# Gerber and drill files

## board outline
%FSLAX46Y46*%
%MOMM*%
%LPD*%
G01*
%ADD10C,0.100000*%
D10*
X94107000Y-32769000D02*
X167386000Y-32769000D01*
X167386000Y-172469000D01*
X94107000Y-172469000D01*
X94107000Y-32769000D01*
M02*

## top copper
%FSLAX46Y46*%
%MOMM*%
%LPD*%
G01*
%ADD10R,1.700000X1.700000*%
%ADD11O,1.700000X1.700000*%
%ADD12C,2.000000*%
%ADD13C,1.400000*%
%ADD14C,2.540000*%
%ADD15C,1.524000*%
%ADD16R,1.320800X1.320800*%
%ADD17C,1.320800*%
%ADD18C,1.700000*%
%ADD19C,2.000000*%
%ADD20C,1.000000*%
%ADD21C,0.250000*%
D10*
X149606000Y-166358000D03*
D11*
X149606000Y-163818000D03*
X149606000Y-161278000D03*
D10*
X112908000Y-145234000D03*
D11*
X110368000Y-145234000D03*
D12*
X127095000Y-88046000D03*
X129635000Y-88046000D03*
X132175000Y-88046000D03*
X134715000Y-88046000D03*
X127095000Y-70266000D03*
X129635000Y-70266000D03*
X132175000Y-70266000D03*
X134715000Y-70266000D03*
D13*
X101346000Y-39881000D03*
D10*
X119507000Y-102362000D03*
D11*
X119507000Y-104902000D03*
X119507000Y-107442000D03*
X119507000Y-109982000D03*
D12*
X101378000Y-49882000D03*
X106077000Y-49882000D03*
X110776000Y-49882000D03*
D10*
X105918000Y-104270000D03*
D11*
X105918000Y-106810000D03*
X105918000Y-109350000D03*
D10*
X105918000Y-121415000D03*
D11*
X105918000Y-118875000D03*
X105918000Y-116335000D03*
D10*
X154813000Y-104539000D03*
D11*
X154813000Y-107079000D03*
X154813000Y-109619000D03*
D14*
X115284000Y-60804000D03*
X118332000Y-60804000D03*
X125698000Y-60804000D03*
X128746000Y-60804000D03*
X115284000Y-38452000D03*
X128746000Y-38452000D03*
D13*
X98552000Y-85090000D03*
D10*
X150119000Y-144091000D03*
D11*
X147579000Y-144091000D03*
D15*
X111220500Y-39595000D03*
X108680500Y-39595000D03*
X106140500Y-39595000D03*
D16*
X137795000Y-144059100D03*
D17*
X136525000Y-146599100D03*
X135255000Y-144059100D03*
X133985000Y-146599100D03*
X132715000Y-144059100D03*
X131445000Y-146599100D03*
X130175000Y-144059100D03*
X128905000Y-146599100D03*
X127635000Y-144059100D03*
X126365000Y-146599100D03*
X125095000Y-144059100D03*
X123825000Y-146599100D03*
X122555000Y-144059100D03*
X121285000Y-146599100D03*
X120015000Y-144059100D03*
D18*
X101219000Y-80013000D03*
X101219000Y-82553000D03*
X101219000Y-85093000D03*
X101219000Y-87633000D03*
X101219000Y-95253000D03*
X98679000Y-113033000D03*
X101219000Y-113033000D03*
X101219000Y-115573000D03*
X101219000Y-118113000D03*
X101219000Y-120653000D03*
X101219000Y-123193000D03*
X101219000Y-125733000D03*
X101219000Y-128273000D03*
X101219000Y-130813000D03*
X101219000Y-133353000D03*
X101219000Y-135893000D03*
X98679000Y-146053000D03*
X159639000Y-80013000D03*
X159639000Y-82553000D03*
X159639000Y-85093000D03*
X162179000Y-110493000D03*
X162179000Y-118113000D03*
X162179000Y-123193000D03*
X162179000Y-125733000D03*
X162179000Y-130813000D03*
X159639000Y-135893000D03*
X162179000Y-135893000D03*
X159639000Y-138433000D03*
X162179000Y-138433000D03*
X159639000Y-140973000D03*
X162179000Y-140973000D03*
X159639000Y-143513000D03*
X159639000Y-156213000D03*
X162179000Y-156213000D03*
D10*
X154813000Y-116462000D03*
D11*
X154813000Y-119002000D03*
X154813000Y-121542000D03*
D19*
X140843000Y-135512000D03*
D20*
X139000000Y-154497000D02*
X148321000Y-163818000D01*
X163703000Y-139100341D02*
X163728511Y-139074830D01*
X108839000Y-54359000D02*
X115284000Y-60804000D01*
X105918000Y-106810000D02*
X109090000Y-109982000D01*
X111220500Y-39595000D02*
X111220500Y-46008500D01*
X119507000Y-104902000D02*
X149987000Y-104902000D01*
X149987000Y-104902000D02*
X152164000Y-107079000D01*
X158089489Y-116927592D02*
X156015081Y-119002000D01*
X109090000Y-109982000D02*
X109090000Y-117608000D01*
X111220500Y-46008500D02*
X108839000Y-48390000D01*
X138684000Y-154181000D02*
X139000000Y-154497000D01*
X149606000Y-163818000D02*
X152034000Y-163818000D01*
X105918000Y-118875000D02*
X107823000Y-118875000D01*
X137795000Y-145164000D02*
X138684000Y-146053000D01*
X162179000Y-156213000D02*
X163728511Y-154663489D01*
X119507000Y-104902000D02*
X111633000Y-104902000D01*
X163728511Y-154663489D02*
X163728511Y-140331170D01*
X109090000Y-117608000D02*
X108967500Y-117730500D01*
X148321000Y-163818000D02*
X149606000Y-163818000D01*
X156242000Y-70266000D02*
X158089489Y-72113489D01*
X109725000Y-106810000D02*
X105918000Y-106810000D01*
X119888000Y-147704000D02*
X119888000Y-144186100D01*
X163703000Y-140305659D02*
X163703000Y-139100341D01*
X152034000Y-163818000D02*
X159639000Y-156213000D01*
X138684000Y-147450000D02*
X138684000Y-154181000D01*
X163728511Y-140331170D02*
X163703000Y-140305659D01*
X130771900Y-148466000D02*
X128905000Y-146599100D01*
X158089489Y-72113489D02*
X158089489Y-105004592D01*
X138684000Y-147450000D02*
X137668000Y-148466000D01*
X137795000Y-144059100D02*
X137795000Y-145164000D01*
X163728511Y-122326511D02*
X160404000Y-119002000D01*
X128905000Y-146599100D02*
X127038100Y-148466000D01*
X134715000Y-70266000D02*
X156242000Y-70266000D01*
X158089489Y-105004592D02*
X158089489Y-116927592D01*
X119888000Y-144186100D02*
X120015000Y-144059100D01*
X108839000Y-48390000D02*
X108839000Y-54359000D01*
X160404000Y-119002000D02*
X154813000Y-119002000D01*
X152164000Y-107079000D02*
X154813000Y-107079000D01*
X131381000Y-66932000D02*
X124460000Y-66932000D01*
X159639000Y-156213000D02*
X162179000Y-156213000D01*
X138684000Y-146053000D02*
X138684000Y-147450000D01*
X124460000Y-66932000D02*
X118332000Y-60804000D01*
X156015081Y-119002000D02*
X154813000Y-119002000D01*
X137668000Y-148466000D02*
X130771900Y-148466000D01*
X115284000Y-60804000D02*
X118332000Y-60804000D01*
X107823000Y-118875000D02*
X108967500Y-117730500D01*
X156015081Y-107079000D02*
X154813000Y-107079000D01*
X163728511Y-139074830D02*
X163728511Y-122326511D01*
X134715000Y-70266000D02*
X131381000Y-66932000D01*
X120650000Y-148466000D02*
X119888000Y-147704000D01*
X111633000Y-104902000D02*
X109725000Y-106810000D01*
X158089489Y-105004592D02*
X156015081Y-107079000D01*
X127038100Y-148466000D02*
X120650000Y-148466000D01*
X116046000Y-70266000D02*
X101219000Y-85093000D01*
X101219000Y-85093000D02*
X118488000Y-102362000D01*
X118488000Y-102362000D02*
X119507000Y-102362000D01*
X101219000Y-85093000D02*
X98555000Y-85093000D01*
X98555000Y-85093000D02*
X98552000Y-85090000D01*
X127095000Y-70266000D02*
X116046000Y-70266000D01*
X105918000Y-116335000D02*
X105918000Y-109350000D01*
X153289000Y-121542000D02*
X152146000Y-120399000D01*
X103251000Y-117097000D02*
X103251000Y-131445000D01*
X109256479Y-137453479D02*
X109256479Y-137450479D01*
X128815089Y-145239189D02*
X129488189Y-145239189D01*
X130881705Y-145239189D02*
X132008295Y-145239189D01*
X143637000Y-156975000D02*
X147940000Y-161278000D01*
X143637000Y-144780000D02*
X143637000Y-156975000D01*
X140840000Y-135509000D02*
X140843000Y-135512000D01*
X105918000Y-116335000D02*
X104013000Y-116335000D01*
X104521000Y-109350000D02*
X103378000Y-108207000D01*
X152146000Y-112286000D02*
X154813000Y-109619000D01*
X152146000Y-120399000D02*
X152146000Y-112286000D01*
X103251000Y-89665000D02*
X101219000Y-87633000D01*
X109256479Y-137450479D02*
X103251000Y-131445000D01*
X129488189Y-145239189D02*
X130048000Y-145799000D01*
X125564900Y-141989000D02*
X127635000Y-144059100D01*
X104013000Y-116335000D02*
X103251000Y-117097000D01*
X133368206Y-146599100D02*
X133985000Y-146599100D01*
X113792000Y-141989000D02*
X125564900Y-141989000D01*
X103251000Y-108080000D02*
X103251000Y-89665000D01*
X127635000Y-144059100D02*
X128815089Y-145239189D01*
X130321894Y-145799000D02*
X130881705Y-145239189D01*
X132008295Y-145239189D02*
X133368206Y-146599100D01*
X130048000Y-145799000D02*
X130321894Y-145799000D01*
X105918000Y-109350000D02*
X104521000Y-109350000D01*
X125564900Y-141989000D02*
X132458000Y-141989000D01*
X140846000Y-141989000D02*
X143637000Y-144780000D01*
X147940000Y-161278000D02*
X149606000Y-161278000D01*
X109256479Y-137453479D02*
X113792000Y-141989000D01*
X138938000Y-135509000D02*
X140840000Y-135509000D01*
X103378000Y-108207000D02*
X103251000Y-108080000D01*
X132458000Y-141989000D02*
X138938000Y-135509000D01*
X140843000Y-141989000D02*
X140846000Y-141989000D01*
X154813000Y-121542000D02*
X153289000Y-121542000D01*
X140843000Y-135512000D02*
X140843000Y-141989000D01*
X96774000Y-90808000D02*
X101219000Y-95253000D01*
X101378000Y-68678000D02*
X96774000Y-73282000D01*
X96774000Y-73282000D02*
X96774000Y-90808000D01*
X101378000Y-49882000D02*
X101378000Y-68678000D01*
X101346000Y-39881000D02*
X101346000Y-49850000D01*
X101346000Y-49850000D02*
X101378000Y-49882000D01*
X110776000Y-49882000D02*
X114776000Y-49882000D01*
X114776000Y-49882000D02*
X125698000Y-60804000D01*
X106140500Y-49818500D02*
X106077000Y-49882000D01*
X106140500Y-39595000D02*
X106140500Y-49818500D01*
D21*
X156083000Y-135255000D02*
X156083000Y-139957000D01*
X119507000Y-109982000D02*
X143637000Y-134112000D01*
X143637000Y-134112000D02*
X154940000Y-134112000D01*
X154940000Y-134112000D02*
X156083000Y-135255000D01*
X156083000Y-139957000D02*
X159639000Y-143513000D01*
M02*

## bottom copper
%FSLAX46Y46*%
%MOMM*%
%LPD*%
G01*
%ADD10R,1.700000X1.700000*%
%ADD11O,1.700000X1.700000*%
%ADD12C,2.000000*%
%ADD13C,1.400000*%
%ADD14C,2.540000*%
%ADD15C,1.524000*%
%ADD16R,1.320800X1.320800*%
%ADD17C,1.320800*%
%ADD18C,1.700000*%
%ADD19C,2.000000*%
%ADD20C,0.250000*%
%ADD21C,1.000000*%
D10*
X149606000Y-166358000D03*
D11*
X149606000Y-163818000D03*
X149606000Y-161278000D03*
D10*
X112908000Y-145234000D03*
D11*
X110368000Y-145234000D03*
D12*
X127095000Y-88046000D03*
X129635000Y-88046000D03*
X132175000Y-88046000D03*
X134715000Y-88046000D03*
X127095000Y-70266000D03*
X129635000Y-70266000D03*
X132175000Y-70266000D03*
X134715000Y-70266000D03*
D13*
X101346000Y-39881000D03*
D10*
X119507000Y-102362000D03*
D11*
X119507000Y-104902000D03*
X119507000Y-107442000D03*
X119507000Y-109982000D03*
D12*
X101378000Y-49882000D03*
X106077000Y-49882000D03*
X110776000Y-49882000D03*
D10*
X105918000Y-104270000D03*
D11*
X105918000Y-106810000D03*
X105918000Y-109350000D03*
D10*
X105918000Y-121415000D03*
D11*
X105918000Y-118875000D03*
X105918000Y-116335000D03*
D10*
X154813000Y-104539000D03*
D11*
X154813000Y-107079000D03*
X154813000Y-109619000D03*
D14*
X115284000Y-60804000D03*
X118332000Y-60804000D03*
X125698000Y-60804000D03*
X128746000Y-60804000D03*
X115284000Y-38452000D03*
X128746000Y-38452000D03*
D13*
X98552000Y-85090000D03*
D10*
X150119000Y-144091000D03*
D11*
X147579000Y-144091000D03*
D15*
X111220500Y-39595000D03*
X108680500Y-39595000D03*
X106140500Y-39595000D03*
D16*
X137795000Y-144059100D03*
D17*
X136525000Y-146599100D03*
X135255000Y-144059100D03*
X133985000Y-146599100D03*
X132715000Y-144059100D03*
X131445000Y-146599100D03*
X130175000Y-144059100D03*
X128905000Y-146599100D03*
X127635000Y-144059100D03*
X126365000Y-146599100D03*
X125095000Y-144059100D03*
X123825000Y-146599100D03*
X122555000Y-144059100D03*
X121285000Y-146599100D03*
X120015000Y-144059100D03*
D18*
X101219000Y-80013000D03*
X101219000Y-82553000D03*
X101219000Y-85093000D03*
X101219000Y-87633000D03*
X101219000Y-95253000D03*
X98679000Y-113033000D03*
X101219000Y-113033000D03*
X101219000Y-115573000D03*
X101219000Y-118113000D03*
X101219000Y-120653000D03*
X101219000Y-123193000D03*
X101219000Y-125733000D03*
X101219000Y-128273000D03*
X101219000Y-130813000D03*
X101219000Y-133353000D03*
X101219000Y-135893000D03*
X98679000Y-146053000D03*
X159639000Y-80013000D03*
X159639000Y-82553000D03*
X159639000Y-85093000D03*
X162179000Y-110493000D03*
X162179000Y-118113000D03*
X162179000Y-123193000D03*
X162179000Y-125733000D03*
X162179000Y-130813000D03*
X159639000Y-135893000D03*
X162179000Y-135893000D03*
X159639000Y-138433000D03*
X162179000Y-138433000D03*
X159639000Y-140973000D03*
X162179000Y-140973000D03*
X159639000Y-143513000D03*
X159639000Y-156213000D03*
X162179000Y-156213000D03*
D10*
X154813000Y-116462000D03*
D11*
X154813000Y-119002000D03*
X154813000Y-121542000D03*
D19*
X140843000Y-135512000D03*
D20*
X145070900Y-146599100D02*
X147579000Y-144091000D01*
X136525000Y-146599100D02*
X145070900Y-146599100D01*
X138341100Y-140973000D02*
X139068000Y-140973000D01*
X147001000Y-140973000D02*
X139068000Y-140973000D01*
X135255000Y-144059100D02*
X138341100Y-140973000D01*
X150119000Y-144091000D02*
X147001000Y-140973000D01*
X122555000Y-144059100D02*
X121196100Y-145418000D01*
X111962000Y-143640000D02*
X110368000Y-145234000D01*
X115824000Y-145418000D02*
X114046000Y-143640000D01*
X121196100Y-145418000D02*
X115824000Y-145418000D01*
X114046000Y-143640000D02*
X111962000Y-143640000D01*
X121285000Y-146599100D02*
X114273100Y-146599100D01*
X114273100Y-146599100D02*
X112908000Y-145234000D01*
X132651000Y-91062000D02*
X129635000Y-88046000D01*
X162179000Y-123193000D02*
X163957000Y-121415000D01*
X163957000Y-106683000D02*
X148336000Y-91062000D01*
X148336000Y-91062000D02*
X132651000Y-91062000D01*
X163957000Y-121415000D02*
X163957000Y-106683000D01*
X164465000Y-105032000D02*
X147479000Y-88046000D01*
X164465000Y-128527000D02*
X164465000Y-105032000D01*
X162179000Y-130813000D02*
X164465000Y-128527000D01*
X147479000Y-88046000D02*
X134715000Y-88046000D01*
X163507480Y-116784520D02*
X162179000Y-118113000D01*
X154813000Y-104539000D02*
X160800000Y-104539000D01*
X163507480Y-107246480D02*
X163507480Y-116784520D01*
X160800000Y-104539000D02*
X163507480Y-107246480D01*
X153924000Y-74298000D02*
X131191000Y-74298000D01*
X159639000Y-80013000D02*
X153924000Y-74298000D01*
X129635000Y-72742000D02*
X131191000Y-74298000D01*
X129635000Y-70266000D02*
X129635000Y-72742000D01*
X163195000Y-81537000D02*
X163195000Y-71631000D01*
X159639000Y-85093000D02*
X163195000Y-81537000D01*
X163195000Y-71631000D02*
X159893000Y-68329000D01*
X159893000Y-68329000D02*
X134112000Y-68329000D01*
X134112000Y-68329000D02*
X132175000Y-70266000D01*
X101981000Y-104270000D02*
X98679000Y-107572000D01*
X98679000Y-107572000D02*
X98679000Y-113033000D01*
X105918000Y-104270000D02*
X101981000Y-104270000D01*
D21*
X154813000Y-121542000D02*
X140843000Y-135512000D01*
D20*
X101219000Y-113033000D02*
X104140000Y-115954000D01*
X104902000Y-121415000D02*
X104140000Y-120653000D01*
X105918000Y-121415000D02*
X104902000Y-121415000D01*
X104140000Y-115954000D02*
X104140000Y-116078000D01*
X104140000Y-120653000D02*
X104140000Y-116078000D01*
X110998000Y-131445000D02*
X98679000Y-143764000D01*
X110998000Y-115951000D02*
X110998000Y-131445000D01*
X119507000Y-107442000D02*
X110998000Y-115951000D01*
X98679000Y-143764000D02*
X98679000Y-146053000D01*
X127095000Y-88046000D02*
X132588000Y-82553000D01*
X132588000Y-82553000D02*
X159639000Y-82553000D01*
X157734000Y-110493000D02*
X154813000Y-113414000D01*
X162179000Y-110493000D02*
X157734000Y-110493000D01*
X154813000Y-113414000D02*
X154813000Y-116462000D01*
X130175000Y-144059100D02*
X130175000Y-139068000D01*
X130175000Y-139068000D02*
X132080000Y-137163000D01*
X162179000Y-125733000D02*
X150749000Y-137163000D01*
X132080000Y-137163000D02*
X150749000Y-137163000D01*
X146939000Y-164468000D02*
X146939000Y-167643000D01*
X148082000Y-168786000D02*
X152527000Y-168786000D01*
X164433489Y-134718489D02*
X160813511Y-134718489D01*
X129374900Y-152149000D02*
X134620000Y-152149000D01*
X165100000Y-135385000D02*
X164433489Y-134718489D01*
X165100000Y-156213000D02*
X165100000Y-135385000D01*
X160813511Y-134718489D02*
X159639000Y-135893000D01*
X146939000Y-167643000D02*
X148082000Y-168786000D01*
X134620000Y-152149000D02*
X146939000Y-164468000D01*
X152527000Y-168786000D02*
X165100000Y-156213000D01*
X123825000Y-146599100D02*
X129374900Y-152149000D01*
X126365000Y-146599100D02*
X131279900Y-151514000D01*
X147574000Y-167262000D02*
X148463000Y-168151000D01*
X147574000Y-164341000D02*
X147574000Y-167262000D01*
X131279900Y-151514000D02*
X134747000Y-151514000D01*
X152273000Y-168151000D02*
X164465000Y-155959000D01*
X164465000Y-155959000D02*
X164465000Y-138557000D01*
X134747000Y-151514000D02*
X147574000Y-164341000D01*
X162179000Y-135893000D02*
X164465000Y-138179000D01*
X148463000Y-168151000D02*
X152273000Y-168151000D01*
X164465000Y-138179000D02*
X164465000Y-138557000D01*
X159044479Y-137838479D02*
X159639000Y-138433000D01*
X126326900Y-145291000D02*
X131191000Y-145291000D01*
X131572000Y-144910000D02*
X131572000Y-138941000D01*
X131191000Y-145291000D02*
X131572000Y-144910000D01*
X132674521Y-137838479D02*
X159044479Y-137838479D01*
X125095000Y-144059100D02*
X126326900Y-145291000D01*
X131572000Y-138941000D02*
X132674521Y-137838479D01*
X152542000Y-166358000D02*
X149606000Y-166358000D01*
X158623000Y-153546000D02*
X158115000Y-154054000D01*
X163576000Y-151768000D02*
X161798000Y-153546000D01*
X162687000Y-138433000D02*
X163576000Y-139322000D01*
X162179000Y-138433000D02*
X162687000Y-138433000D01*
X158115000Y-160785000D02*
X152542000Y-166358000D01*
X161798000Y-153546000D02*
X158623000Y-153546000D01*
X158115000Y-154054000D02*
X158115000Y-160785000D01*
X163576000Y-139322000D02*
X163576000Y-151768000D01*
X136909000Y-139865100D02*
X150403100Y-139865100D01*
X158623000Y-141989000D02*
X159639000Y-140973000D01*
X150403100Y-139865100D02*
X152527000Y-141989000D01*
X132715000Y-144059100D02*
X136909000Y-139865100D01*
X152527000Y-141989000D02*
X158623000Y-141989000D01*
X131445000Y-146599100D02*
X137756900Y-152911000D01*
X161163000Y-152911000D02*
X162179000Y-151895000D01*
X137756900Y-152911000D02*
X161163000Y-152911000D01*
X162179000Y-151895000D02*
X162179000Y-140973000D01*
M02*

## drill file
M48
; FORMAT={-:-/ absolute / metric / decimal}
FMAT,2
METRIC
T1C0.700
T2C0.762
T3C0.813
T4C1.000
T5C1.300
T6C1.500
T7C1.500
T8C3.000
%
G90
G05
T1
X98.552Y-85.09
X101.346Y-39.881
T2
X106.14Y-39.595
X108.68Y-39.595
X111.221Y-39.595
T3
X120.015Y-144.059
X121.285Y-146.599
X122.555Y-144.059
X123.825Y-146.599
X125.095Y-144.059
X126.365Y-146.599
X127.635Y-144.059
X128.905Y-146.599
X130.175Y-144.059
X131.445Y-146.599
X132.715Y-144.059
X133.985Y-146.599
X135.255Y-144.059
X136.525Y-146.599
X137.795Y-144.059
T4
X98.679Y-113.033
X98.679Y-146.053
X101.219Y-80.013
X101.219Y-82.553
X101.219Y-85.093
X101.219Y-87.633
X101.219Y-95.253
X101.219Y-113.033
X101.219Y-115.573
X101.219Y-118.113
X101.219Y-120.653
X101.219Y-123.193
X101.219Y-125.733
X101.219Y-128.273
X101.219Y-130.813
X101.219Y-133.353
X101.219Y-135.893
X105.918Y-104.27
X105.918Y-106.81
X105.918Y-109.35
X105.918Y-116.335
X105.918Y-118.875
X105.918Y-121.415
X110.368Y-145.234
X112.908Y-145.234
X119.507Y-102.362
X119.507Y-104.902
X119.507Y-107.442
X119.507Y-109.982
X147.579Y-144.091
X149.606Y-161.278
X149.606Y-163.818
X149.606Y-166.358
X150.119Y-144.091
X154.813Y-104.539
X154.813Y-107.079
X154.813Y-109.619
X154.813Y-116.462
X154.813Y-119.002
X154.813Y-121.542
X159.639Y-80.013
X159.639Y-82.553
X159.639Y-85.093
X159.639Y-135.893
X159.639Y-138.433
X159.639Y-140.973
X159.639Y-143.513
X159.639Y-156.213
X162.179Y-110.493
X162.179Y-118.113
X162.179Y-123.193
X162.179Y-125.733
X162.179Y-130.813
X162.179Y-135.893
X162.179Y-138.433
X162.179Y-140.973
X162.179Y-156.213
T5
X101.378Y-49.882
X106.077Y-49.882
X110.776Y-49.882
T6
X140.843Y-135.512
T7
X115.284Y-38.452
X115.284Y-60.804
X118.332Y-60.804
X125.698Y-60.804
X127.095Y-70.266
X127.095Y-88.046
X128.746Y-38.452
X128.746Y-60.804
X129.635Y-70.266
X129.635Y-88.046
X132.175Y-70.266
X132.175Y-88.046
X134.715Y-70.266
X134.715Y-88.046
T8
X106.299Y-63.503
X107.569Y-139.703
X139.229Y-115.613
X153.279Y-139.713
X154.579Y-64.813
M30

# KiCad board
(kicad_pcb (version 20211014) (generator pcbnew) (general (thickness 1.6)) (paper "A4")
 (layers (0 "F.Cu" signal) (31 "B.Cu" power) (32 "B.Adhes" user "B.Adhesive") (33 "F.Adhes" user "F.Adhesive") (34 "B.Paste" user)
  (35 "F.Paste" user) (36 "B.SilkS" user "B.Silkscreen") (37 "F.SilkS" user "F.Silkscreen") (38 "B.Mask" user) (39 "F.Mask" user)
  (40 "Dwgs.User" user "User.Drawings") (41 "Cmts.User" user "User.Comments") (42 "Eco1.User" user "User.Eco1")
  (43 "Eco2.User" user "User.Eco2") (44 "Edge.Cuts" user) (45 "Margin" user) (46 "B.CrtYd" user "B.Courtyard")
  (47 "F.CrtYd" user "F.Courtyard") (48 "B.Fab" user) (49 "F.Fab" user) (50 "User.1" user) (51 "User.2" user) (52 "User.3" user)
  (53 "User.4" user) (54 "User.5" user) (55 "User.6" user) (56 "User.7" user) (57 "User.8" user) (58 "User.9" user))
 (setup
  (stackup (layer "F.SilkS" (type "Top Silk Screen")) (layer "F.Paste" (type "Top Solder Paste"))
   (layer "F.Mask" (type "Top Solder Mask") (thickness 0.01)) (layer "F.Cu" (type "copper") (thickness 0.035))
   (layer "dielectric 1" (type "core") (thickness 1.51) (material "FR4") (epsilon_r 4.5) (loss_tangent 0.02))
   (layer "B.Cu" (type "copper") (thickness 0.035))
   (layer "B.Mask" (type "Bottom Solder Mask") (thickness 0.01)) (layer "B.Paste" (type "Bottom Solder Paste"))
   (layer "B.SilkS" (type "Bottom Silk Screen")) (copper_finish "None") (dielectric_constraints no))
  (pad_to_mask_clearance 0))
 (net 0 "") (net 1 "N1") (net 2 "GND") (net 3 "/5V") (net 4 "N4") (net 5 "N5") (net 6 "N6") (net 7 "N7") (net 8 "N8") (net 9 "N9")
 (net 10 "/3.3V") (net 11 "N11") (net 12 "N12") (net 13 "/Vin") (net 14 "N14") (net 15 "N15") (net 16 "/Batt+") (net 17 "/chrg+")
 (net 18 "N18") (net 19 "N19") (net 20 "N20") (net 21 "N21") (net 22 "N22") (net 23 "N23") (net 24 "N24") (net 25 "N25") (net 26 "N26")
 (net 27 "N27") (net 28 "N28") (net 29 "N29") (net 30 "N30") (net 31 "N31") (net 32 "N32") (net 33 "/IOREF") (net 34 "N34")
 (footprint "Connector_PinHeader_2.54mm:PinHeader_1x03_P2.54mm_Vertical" (layer "F.Cu") (at 149.606 166.358 180)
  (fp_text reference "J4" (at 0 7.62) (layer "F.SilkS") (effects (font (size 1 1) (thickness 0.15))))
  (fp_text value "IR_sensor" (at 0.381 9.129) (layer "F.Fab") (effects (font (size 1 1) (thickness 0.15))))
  (pad "1" thru_hole rect (at 0 0 180) (size 1.7 1.7) (drill 1) (layers *.Cu *.Mask) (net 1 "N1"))
  (pad "2" thru_hole oval (at 0 2.54 180) (size 1.7 1.7) (drill 1) (layers *.Cu *.Mask) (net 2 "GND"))
  (pad "3" thru_hole oval (at 0 5.08 180) (size 1.7 1.7) (drill 1) (layers *.Cu *.Mask) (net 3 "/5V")))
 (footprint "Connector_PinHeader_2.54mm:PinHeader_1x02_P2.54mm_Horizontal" (layer "F.Cu") (at 112.908 145.234 -90)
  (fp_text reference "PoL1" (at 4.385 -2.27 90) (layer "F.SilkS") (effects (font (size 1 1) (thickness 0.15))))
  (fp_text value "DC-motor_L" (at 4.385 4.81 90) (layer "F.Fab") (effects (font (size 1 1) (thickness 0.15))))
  (pad "1" thru_hole rect (at 0 0 270) (size 1.7 1.7) (drill 1) (layers *.Cu *.Mask) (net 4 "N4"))
  (pad "2" thru_hole oval (at 0 2.54 270) (size 1.7 1.7) (drill 1) (layers *.Cu *.Mask) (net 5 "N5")))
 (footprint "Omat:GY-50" (layer "F.Cu") (at 119.348 90.713)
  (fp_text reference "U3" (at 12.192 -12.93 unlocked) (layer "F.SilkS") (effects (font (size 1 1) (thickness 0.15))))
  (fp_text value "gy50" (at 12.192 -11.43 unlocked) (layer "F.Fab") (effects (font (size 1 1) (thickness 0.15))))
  (pad "1" thru_hole circle (at 7.747 -2.667) (size 2 2) (drill 1.5) (layers *.Cu *.Mask) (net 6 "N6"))
  (pad "2" thru_hole circle (at 10.287 -2.667) (size 2 2) (drill 1.5) (layers *.Cu *.Mask) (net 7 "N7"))
  (pad "3" thru_hole circle (at 12.827 -2.667) (size 2 2) (drill 1.5) (layers *.Cu *.Mask) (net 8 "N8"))
  (pad "4" thru_hole circle (at 15.367 -2.667) (size 2 2) (drill 1.5) (layers *.Cu *.Mask) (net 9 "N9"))
  (pad "5" thru_hole circle (at 7.747 -20.447) (size 2 2) (drill 1.5) (layers *.Cu *.Mask) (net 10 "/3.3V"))
  (pad "6" thru_hole circle (at 10.287 -20.447) (size 2 2) (drill 1.5) (layers *.Cu *.Mask) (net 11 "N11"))
  (pad "7" thru_hole circle (at 12.827 -20.447) (size 2 2) (drill 1.5) (layers *.Cu *.Mask) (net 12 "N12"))
  (pad "8" thru_hole circle (at 15.367 -20.447) (size 2 2) (drill 1.5) (layers *.Cu *.Mask) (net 2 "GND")))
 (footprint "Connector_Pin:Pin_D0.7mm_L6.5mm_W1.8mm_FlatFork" (layer "F.Cu") (at 101.346 39.881)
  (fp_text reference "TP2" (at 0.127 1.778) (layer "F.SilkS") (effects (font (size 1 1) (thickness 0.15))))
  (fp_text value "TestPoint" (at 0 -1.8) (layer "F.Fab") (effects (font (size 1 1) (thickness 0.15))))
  (pad "1" thru_hole circle (at 0 0) (size 1.4 1.4) (drill 0.7) (layers *.Cu *.Mask) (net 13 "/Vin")))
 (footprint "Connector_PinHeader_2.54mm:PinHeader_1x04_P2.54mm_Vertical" (layer "F.Cu") (at 119.507 102.362)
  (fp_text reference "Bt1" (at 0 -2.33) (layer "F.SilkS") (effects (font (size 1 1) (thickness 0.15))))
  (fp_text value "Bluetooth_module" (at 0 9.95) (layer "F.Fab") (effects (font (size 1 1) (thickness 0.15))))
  (pad "1" thru_hole rect (at 0 0) (size 1.7 1.7) (drill 1) (layers *.Cu *.Mask) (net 10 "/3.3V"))
  (pad "2" thru_hole oval (at 0 2.54) (size 1.7 1.7) (drill 1) (layers *.Cu *.Mask) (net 2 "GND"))
  (pad "3" thru_hole oval (at 0 5.08) (size 1.7 1.7) (drill 1) (layers *.Cu *.Mask) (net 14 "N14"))
  (pad "4" thru_hole oval (at 0 7.62) (size 1.7 1.7) (drill 1) (layers *.Cu *.Mask) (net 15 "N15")))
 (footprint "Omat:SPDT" (layer "F.Cu") (at 112.681 45.818 180)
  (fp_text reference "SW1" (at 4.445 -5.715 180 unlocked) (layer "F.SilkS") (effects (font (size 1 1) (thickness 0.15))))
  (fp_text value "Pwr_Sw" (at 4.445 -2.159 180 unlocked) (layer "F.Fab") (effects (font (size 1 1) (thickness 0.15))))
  (pad "1" thru_hole circle (at 11.303 -4.064 180) (size 2 2) (drill 1.3) (layers *.Cu *.Mask) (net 13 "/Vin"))
  (pad "2" thru_hole circle (at 6.604 -4.064 180) (size 2 2) (drill 1.3) (layers *.Cu *.Mask) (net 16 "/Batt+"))
  (pad "3" thru_hole circle (at 1.905 -4.064 180) (size 2 2) (drill 1.3) (layers *.Cu *.Mask) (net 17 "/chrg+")))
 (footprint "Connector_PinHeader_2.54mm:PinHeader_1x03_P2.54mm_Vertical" (layer "F.Cu") (at 105.918 104.27)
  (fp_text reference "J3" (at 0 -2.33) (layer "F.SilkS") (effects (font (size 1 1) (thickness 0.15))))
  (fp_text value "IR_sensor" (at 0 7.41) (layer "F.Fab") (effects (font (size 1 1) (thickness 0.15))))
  (pad "1" thru_hole rect (at 0 0) (size 1.7 1.7) (drill 1) (layers *.Cu *.Mask) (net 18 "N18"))
  (pad "2" thru_hole oval (at 0 2.54) (size 1.7 1.7) (drill 1) (layers *.Cu *.Mask) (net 2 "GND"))
  (pad "3" thru_hole oval (at 0 5.08) (size 1.7 1.7) (drill 1) (layers *.Cu *.Mask) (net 3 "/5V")))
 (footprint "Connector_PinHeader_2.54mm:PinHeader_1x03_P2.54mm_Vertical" (layer "F.Cu") (at 105.918 121.415 180)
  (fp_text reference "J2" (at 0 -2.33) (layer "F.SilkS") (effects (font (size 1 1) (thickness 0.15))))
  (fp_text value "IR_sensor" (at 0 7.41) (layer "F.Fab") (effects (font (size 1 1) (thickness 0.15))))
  (pad "1" thru_hole rect (at 0 0 180) (size 1.7 1.7) (drill 1) (layers *.Cu *.Mask) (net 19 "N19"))
  (pad "2" thru_hole oval (at 0 2.54 180) (size 1.7 1.7) (drill 1) (layers *.Cu *.Mask) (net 2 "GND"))
  (pad "3" thru_hole oval (at 0 5.08 180) (size 1.7 1.7) (drill 1) (layers *.Cu *.Mask) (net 3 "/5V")))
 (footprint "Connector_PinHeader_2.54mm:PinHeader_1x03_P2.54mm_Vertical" (layer "F.Cu") (at 154.813 104.539)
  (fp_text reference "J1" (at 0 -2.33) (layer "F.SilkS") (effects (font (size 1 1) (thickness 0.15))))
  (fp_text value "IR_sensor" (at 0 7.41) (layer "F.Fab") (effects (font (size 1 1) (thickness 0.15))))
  (pad "1" thru_hole rect (at 0 0) (size 1.7 1.7) (drill 1) (layers *.Cu *.Mask) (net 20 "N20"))
  (pad "2" thru_hole oval (at 0 2.54) (size 1.7 1.7) (drill 1) (layers *.Cu *.Mask) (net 2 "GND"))
  (pad "3" thru_hole oval (at 0 5.08) (size 1.7 1.7) (drill 1) (layers *.Cu *.Mask) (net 3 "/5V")))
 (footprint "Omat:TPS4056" (layer "F.Cu") (at 113.506 35.912 -90)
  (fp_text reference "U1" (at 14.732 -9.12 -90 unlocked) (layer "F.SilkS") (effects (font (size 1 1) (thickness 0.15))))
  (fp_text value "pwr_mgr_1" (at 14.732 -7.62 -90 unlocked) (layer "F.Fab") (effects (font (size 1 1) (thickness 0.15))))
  (pad "1" thru_hole circle (at 24.892 -1.778 270) (size 2.54 2.54) (drill 1.5) (layers *.Cu *.Mask) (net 2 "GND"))
  (pad "2" thru_hole circle (at 24.892 -4.826 270) (size 2.54 2.54) (drill 1.5) (layers *.Cu *.Mask) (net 2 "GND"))
  (pad "3" thru_hole circle (at 24.892 -12.192 270) (size 2.54 2.54) (drill 1.5) (layers *.Cu *.Mask) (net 17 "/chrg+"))
  (pad "4" thru_hole circle (at 24.892 -15.24 270) (size 2.54 2.54) (drill 1.5) (layers *.Cu *.Mask) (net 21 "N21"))
  (pad "5" thru_hole circle (at 2.54 -1.778 270) (size 2.54 2.54) (drill 1.5) (layers *.Cu *.Mask) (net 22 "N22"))
  (pad "6" thru_hole circle (at 2.54 -15.24 270) (size 2.54 2.54) (drill 1.5) (layers *.Cu *.Mask) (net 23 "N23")))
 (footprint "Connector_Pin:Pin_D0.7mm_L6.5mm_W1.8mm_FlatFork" (layer "F.Cu") (at 98.552 85.09)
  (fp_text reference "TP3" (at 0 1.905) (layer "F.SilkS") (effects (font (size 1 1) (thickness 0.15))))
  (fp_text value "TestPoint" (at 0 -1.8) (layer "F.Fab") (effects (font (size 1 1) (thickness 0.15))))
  (pad "1" thru_hole circle (at 0 0) (size 1.4 1.4) (drill 0.7) (layers *.Cu *.Mask) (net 10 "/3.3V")))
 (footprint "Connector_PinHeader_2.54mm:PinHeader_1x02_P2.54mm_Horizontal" (layer "F.Cu") (at 150.119 144.091 -90)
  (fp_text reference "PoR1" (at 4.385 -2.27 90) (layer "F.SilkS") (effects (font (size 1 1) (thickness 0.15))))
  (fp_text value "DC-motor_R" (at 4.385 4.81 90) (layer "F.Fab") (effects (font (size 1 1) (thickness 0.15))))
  (pad "1" thru_hole rect (at 0 0 270) (size 1.7 1.7) (drill 1) (layers *.Cu *.Mask) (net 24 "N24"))
  (pad "2" thru_hole oval (at 0 2.54 270) (size 1.7 1.7) (drill 1) (layers *.Cu *.Mask) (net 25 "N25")))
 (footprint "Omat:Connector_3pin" (layer "F.Cu") (at 112.3635 38.325 180)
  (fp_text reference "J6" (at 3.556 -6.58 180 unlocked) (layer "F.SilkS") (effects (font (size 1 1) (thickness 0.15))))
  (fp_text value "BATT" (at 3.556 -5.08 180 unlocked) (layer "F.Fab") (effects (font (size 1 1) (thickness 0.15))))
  (pad "1" thru_hole circle (at 1.143 -1.27 180) (size 1.524 1.524) (drill 0.762) (layers *.Cu *.Mask) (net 2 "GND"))
  (pad "2" thru_hole circle (at 3.683 -1.27 180) (size 1.524 1.524) (drill 0.762) (layers *.Cu *.Mask) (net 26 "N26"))
  (pad "3" thru_hole circle (at 6.223 -1.27 180) (size 1.524 1.524) (drill 0.762) (layers *.Cu *.Mask) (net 16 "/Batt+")))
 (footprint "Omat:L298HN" (layer "F.Cu") (at 137.795 144.0591 180)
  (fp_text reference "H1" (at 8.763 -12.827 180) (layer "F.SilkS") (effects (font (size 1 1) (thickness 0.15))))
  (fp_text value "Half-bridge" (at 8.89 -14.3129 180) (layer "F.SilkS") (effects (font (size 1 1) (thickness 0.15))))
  (pad "1" thru_hole rect (at 0 0 180) (size 1.3208 1.3208) (drill 0.8128) (layers *.Cu *.Mask) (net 2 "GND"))
  (pad "2" thru_hole circle (at 1.27 -2.54 180) (size 1.3208 1.3208) (drill 0.8128) (layers *.Cu *.Mask) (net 25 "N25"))
  (pad "3" thru_hole circle (at 2.54 0 180) (size 1.3208 1.3208) (drill 0.8128) (layers *.Cu *.Mask) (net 24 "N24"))
  (pad "4" thru_hole circle (at 3.81 -2.54 180) (size 1.3208 1.3208) (drill 0.8128) (layers *.Cu *.Mask) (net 3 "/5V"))
  (pad "5" thru_hole circle (at 5.08 0 180) (size 1.3208 1.3208) (drill 0.8128) (layers *.Cu *.Mask) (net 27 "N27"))
  (pad "6" thru_hole circle (at 6.35 -2.54 180) (size 1.3208 1.3208) (drill 0.8128) (layers *.Cu *.Mask) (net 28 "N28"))
  (pad "7" thru_hole circle (at 7.62 0 180) (size 1.3208 1.3208) (drill 0.8128) (layers *.Cu *.Mask) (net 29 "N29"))
  (pad "8" thru_hole circle (at 8.89 -2.54 180) (size 1.3208 1.3208) (drill 0.8128) (layers *.Cu *.Mask) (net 2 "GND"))
  (pad "9" thru_hole circle (at 10.16 0 180) (size 1.3208 1.3208) (drill 0.8128) (layers *.Cu *.Mask) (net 3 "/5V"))
  (pad "10" thru_hole circle (at 11.43 -2.54 180) (size 1.3208 1.3208) (drill 0.8128) (layers *.Cu *.Mask) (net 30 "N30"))
  (pad "11" thru_hole circle (at 12.7 0 180) (size 1.3208 1.3208) (drill 0.8128) (layers *.Cu *.Mask) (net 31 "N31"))
  (pad "12" thru_hole circle (at 13.97 -2.54 180) (size 1.3208 1.3208) (drill 0.8128) (layers *.Cu *.Mask) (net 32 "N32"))
  (pad "13" thru_hole circle (at 15.24 0 180) (size 1.3208 1.3208) (drill 0.8128) (layers *.Cu *.Mask) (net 5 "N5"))
  (pad "14" thru_hole circle (at 16.51 -2.54 180) (size 1.3208 1.3208) (drill 0.8128) (layers *.Cu *.Mask) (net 4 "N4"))
  (pad "15" thru_hole circle (at 17.78 0 180) (size 1.3208 1.3208) (drill 0.8128) (layers *.Cu *.Mask) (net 2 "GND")))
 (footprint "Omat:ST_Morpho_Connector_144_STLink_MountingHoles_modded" (layer "F.Cu") (at 98.679 67.313)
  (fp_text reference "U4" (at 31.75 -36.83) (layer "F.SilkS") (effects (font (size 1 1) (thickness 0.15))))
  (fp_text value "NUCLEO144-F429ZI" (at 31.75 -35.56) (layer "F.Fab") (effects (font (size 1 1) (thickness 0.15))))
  (pad "" np_thru_hole circle (at 40.55 48.3) (size 3 3) (drill 3) (layers *.Cu *.Mask))
  (pad "" np_thru_hole circle (at 55.9 -2.5) (size 3 3) (drill 3) (layers *.Cu *.Mask))
  (pad "" np_thru_hole circle (at 8.89 72.39) (size 3 3) (drill 3) (layers *.Cu *.Mask))
  (pad "" np_thru_hole circle (at 7.62 -3.81) (size 3 3) (drill 3) (layers *.Cu *.Mask))
  (pad "" np_thru_hole circle (at 54.6 72.4) (size 3 3) (drill 3) (layers *.Cu *.Mask))
  (pad "12" thru_hole circle (at 2.54 12.7) (size 1.7 1.7) (drill 1) (layers *.Cu *.Mask) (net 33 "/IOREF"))
  (pad "14" thru_hole circle (at 2.54 15.24) (size 1.7 1.7) (drill 1) (layers *.Cu *.Mask))
  (pad "16" thru_hole circle (at 2.54 17.78) (size 1.7 1.7) (drill 1) (layers *.Cu *.Mask) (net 10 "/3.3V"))
  (pad "18" thru_hole circle (at 2.54 20.32) (size 1.7 1.7) (drill 1) (layers *.Cu *.Mask) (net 3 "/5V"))
  (pad "24" thru_hole circle (at 2.54 27.94) (size 1.7 1.7) (drill 1) (layers *.Cu *.Mask) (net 13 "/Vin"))
  (pad "37" thru_hole circle (at 0 45.72) (size 1.7 1.7) (drill 1) (layers *.Cu *.Mask) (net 18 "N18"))
  (pad "38" thru_hole circle (at 2.54 45.72) (size 1.7 1.7) (drill 1) (layers *.Cu *.Mask) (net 19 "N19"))
  (pad "40" thru_hole circle (at 2.54 48.26) (size 1.7 1.7) (drill 1) (layers *.Cu *.Mask))
  (pad "42" thru_hole circle (at 2.54 50.8) (size 1.7 1.7) (drill 1) (layers *.Cu *.Mask))
  (pad "44" thru_hole circle (at 2.54 53.34) (size 1.7 1.7) (drill 1) (layers *.Cu *.Mask))
  (pad "46" thru_hole circle (at 2.54 55.88) (size 1.7 1.7) (drill 1) (layers *.Cu *.Mask))
  (pad "48" thru_hole circle (at 2.54 58.42) (size 1.7 1.7) (drill 1) (layers *.Cu *.Mask))
  (pad "50" thru_hole circle (at 2.54 60.96) (size 1.7 1.7) (drill 1) (layers *.Cu *.Mask))
  (pad "52" thru_hole circle (at 2.54 63.5) (size 1.7 1.7) (drill 1) (layers *.Cu *.Mask))
  (pad "54" thru_hole circle (at 2.54 66.04) (size 1.7 1.7) (drill 1) (layers *.Cu *.Mask))
  (pad "56" thru_hole circle (at 2.54 68.58) (size 1.7 1.7) (drill 1) (layers *.Cu *.Mask))
  (pad "63" thru_hole circle (at 0 78.74) (size 1.7 1.7) (drill 1) (layers *.Cu *.Mask) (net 14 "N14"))
  (pad "83" thru_hole circle (at 60.96 12.7) (size 1.7 1.7) (drill 1) (layers *.Cu *.Mask) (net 11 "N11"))
  (pad "85" thru_hole circle (at 60.96 15.24) (size 1.7 1.7) (drill 1) (layers *.Cu *.Mask) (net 6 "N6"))
  (pad "87" thru_hole circle (at 60.96 17.78) (size 1.7 1.7) (drill 1) (layers *.Cu *.Mask) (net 12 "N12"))
  (pad "108" thru_hole circle (at 63.5 43.18) (size 1.7 1.7) (drill 1) (layers *.Cu *.Mask) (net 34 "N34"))
  (pad "114" thru_hole circle (at 63.5 50.8) (size 1.7 1.7) (drill 1) (layers *.Cu *.Mask) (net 20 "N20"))
  (pad "118" thru_hole circle (at 63.5 55.88) (size 1.7 1.7) (drill 1) (layers *.Cu *.Mask) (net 7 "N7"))
  (pad "120" thru_hole circle (at 63.5 58.42) (size 1.7 1.7) (drill 1) (layers *.Cu *.Mask) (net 29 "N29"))
  (pad "124" thru_hole circle (at 63.5 63.5) (size 1.7 1.7) (drill 1) (layers *.Cu *.Mask) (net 9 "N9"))
  (pad "127" thru_hole circle (at 60.96 68.58) (size 1.7 1.7) (drill 1) (layers *.Cu *.Mask) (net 32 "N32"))
  (pad "128" thru_hole circle (at 63.5 68.58) (size 1.7 1.7) (drill 1) (layers *.Cu *.Mask) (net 30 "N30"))
  (pad "129" thru_hole circle (at 60.96 71.12) (size 1.7 1.7) (drill 1) (layers *.Cu *.Mask) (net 31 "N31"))
  (pad "130" thru_hole circle (at 63.5 71.12) (size 1.7 1.7) (drill 1) (layers *.Cu *.Mask) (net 1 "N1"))
  (pad "131" thru_hole circle (at 60.96 73.66) (size 1.7 1.7) (drill 1) (layers *.Cu *.Mask) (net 27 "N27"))
  (pad "132" thru_hole circle (at 63.5 73.66) (size 1.7 1.7) (drill 1) (layers *.Cu *.Mask) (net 28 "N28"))
  (pad "133" thru_hole circle (at 60.96 76.2) (size 1.7 1.7) (drill 1) (layers *.Cu *.Mask) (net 15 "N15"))
  (pad "143" thru_hole circle (at 60.96 88.9) (size 1.7 1.7) (drill 1) (layers *.Cu *.Mask) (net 2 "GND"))
  (pad "144" thru_hole circle (at 63.5 88.9) (size 1.7 1.7) (drill 1) (layers *.Cu *.Mask) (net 2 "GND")))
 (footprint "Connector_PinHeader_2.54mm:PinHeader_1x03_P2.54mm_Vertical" (layer "F.Cu") (at 154.813 116.462)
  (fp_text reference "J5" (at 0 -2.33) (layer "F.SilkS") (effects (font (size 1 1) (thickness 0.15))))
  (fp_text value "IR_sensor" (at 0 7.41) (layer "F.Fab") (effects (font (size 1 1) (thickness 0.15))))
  (pad "1" thru_hole rect (at 0 0) (size 1.7 1.7) (drill 1) (layers *.Cu *.Mask) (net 34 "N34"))
  (pad "2" thru_hole oval (at 0 2.54) (size 1.7 1.7) (drill 1) (layers *.Cu *.Mask) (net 2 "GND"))
  (pad "3" thru_hole oval (at 0 5.08) (size 1.7 1.7) (drill 1) (layers *.Cu *.Mask) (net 3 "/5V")))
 (gr_rect (start 94.107 32.769) (end 167.386 172.469) (layer "Edge.Cuts") (width 0.1) (fill none))
 (segment (start 139 154.497) (end 148.321 163.818) (width 1) (layer "F.Cu") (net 2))
 (segment (start 163.703 139.100341) (end 163.728511 139.07483) (width 1) (layer "F.Cu") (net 2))
 (segment (start 108.839 54.359) (end 115.284 60.804) (width 1) (layer "F.Cu") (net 2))
 (segment (start 105.918 106.81) (end 109.09 109.982) (width 1) (layer "F.Cu") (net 2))
 (segment (start 111.2205 39.595) (end 111.2205 46.0085) (width 1) (layer "F.Cu") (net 2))
 (segment (start 119.507 104.902) (end 149.987 104.902) (width 1) (layer "F.Cu") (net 2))
 (segment (start 149.987 104.902) (end 152.164 107.079) (width 1) (layer "F.Cu") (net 2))
 (segment (start 158.089489 116.927592) (end 156.015081 119.002) (width 1) (layer "F.Cu") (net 2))
 (segment (start 109.09 109.982) (end 109.09 117.608) (width 1) (layer "F.Cu") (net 2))
 (segment (start 111.2205 46.0085) (end 108.839 48.39) (width 1) (layer "F.Cu") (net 2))
 (segment (start 138.684 154.181) (end 139 154.497) (width 1) (layer "F.Cu") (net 2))
 (segment (start 149.606 163.818) (end 152.034 163.818) (width 1) (layer "F.Cu") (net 2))
 (segment (start 105.918 118.875) (end 107.823 118.875) (width 1) (layer "F.Cu") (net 2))
 (segment (start 137.795 145.164) (end 138.684 146.053) (width 1) (layer "F.Cu") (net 2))
 (segment (start 162.179 156.213) (end 163.728511 154.663489) (width 1) (layer "F.Cu") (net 2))
 (segment (start 119.507 104.902) (end 111.633 104.902) (width 1) (layer "F.Cu") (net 2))
 (segment (start 163.728511 154.663489) (end 163.728511 140.33117) (width 1) (layer "F.Cu") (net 2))
 (segment (start 109.09 117.608) (end 108.9675 117.7305) (width 1) (layer "F.Cu") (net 2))
 (segment (start 148.321 163.818) (end 149.606 163.818) (width 1) (layer "F.Cu") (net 2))
 (segment (start 156.242 70.266) (end 158.089489 72.113489) (width 1) (layer "F.Cu") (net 2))
 (segment (start 109.725 106.81) (end 105.918 106.81) (width 1) (layer "F.Cu") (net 2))
 (segment (start 119.888 147.704) (end 119.888 144.1861) (width 1) (layer "F.Cu") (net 2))
 (segment (start 163.703 140.305659) (end 163.703 139.100341) (width 1) (layer "F.Cu") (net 2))
 (segment (start 152.034 163.818) (end 159.639 156.213) (width 1) (layer "F.Cu") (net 2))
 (segment (start 138.684 147.45) (end 138.684 154.181) (width 1) (layer "F.Cu") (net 2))
 (segment (start 163.728511 140.33117) (end 163.703 140.305659) (width 1) (layer "F.Cu") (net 2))
 (segment (start 130.7719 148.466) (end 128.905 146.5991) (width 1) (layer "F.Cu") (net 2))
 (segment (start 158.089489 72.113489) (end 158.089489 105.004592) (width 1) (layer "F.Cu") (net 2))
 (segment (start 138.684 147.45) (end 137.668 148.466) (width 1) (layer "F.Cu") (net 2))
 (segment (start 137.795 144.0591) (end 137.795 145.164) (width 1) (layer "F.Cu") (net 2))
 (segment (start 163.728511 122.326511) (end 160.404 119.002) (width 1) (layer "F.Cu") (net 2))
 (segment (start 128.905 146.5991) (end 127.0381 148.466) (width 1) (layer "F.Cu") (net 2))
 (segment (start 134.715 70.266) (end 156.242 70.266) (width 1) (layer "F.Cu") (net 2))
 (segment (start 158.089489 105.004592) (end 158.089489 116.927592) (width 1) (layer "F.Cu") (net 2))
 (segment (start 119.888 144.1861) (end 120.015 144.0591) (width 1) (layer "F.Cu") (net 2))
 (segment (start 108.839 48.39) (end 108.839 54.359) (width 1) (layer "F.Cu") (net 2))
 (segment (start 160.404 119.002) (end 154.813 119.002) (width 1) (layer "F.Cu") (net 2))
 (segment (start 152.164 107.079) (end 154.813 107.079) (width 1) (layer "F.Cu") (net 2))
 (segment (start 131.381 66.932) (end 124.46 66.932) (width 1) (layer "F.Cu") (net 2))
 (segment (start 159.639 156.213) (end 162.179 156.213) (width 1) (layer "F.Cu") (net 2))
 (segment (start 138.684 146.053) (end 138.684 147.45) (width 1) (layer "F.Cu") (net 2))
 (segment (start 124.46 66.932) (end 118.332 60.804) (width 1) (layer "F.Cu") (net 2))
 (segment (start 156.015081 119.002) (end 154.813 119.002) (width 1) (layer "F.Cu") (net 2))
 (segment (start 137.668 148.466) (end 130.7719 148.466) (width 1) (layer "F.Cu") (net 2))
 (segment (start 115.284 60.804) (end 118.332 60.804) (width 1) (layer "F.Cu") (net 2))
 (segment (start 107.823 118.875) (end 108.9675 117.7305) (width 1) (layer "F.Cu") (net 2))
 (segment (start 156.015081 107.079) (end 154.813 107.079) (width 1) (layer "F.Cu") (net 2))
 (segment (start 163.728511 139.07483) (end 163.728511 122.326511) (width 1) (layer "F.Cu") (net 2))
 (segment (start 134.715 70.266) (end 131.381 66.932) (width 1) (layer "F.Cu") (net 2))
 (segment (start 120.65 148.466) (end 119.888 147.704) (width 1) (layer "F.Cu") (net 2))
 (segment (start 111.633 104.902) (end 109.725 106.81) (width 1) (layer "F.Cu") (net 2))
 (segment (start 158.089489 105.004592) (end 156.015081 107.079) (width 1) (layer "F.Cu") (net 2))
 (segment (start 127.0381 148.466) (end 120.65 148.466) (width 1) (layer "F.Cu") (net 2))
 (segment (start 145.0709 146.5991) (end 147.579 144.091) (width 0.25) (layer "B.Cu") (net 25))
 (segment (start 136.525 146.5991) (end 145.0709 146.5991) (width 0.25) (layer "B.Cu") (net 25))
 (segment (start 138.3411 140.973) (end 139.068 140.973) (width 0.25) (layer "B.Cu") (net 24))
 (segment (start 147.001 140.973) (end 139.068 140.973) (width 0.25) (layer "B.Cu") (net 24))
 (segment (start 135.255 144.0591) (end 138.3411 140.973) (width 0.25) (layer "B.Cu") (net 24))
 (segment (start 150.119 144.091) (end 147.001 140.973) (width 0.25) (layer "B.Cu") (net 24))
 (segment (start 116.046 70.266) (end 101.219 85.093) (width 1) (layer "F.Cu") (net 10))
 (segment (start 101.219 85.093) (end 118.488 102.362) (width 1) (layer "F.Cu") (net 10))
 (segment (start 118.488 102.362) (end 119.507 102.362) (width 1) (layer "F.Cu") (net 10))
 (segment (start 101.219 85.093) (end 98.555 85.093) (width 1) (layer "F.Cu") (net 10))
 (segment (start 98.555 85.093) (end 98.552 85.09) (width 1) (layer "F.Cu") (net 10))
 (segment (start 127.095 70.266) (end 116.046 70.266) (width 1) (layer "F.Cu") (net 10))
 (segment (start 122.555 144.0591) (end 121.1961 145.418) (width 0.25) (layer "B.Cu") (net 5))
 (segment (start 111.962 143.64) (end 110.368 145.234) (width 0.25) (layer "B.Cu") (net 5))
 (segment (start 115.824 145.418) (end 114.046 143.64) (width 0.25) (layer "B.Cu") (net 5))
 (segment (start 121.1961 145.418) (end 115.824 145.418) (width 0.25) (layer "B.Cu") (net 5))
 (segment (start 114.046 143.64) (end 111.962 143.64) (width 0.25) (layer "B.Cu") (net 5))
 (segment (start 121.285 146.5991) (end 114.2731 146.5991) (width 0.25) (layer "B.Cu") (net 4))
 (segment (start 114.2731 146.5991) (end 112.908 145.234) (width 0.25) (layer "B.Cu") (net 4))
 (segment (start 132.651 91.062) (end 129.635 88.046) (width 0.25) (layer "B.Cu") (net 7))
 (segment (start 162.179 123.193) (end 163.957 121.415) (width 0.25) (layer "B.Cu") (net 7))
 (segment (start 163.957 106.683) (end 148.336 91.062) (width 0.25) (layer "B.Cu") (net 7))
 (segment (start 148.336 91.062) (end 132.651 91.062) (width 0.25) (layer "B.Cu") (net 7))
 (segment (start 163.957 121.415) (end 163.957 106.683) (width 0.25) (layer "B.Cu") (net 7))
 (segment (start 164.465 105.032) (end 147.479 88.046) (width 0.25) (layer "B.Cu") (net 9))
 (segment (start 164.465 128.527) (end 164.465 105.032) (width 0.25) (layer "B.Cu") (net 9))
 (segment (start 162.179 130.813) (end 164.465 128.527) (width 0.25) (layer "B.Cu") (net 9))
 (segment (start 147.479 88.046) (end 134.715 88.046) (width 0.25) (layer "B.Cu") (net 9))
 (segment (start 163.50748 116.78452) (end 162.179 118.113) (width 0.25) (layer "B.Cu") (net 20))
 (segment (start 154.813 104.539) (end 160.8 104.539) (width 0.25) (layer "B.Cu") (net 20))
 (segment (start 163.50748 107.24648) (end 163.50748 116.78452) (width 0.25) (layer "B.Cu") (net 20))
 (segment (start 160.8 104.539) (end 163.50748 107.24648) (width 0.25) (layer "B.Cu") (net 20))
 (segment (start 153.924 74.298) (end 131.191 74.298) (width 0.25) (layer "B.Cu") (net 11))
 (segment (start 159.639 80.013) (end 153.924 74.298) (width 0.25) (layer "B.Cu") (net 11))
 (segment (start 129.635 72.742) (end 131.191 74.298) (width 0.25) (layer "B.Cu") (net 11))
 (segment (start 129.635 70.266) (end 129.635 72.742) (width 0.25) (layer "B.Cu") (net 11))
 (segment (start 163.195 81.537) (end 163.195 71.631) (width 0.25) (layer "B.Cu") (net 12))
 (segment (start 159.639 85.093) (end 163.195 81.537) (width 0.25) (layer "B.Cu") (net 12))
 (segment (start 163.195 71.631) (end 159.893 68.329) (width 0.25) (layer "B.Cu") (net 12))
 (segment (start 159.893 68.329) (end 134.112 68.329) (width 0.25) (layer "B.Cu") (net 12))
 (segment (start 134.112 68.329) (end 132.175 70.266) (width 0.25) (layer "B.Cu") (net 12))
 (segment (start 101.981 104.27) (end 98.679 107.572) (width 0.25) (layer "B.Cu") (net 18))
 (segment (start 98.679 107.572) (end 98.679 113.033) (width 0.25) (layer "B.Cu") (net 18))
 (segment (start 105.918 104.27) (end 101.981 104.27) (width 0.25) (layer "B.Cu") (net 18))
 (segment (start 105.918 116.335) (end 105.918 109.35) (width 1) (layer "F.Cu") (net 3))
 (segment (start 153.289 121.542) (end 152.146 120.399) (width 1) (layer "F.Cu") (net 3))
 (segment (start 103.251 117.097) (end 103.251 131.445) (width 1) (layer "F.Cu") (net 3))
 (segment (start 109.256479 137.453479) (end 109.256479 137.450479) (width 1) (layer "F.Cu") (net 3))
 (segment (start 128.815089 145.239189) (end 129.488189 145.239189) (width 1) (layer "F.Cu") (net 3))
 (segment (start 130.881705 145.239189) (end 132.008295 145.239189) (width 1) (layer "F.Cu") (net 3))
 (segment (start 143.637 156.975) (end 147.94 161.278) (width 1) (layer "F.Cu") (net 3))
 (segment (start 143.637 144.78) (end 143.637 156.975) (width 1) (layer "F.Cu") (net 3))
 (segment (start 140.84 135.509) (end 140.843 135.512) (width 1) (layer "F.Cu") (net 3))
 (segment (start 105.918 116.335) (end 104.013 116.335) (width 1) (layer "F.Cu") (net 3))
 (segment (start 104.521 109.35) (end 103.378 108.207) (width 1) (layer "F.Cu") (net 3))
 (segment (start 152.146 112.286) (end 154.813 109.619) (width 1) (layer "F.Cu") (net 3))
 (segment (start 152.146 120.399) (end 152.146 112.286) (width 1) (layer "F.Cu") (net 3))
 (segment (start 103.251 89.665) (end 101.219 87.633) (width 1) (layer "F.Cu") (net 3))
 (segment (start 109.256479 137.450479) (end 103.251 131.445) (width 1) (layer "F.Cu") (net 3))
 (segment (start 129.488189 145.239189) (end 130.048 145.799) (width 1) (layer "F.Cu") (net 3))
 (segment (start 125.5649 141.989) (end 127.635 144.0591) (width 1) (layer "F.Cu") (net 3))
 (segment (start 104.013 116.335) (end 103.251 117.097) (width 1) (layer "F.Cu") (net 3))
 (segment (start 133.368206 146.5991) (end 133.985 146.5991) (width 1) (layer "F.Cu") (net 3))
 (segment (start 113.792 141.989) (end 125.5649 141.989) (width 1) (layer "F.Cu") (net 3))
 (segment (start 103.251 108.08) (end 103.251 89.665) (width 1) (layer "F.Cu") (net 3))
 (segment (start 127.635 144.0591) (end 128.815089 145.239189) (width 1) (layer "F.Cu") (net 3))
 (segment (start 130.321894 145.799) (end 130.881705 145.239189) (width 1) (layer "F.Cu") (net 3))
 (segment (start 132.008295 145.239189) (end 133.368206 146.5991) (width 1) (layer "F.Cu") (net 3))
 (segment (start 130.048 145.799) (end 130.321894 145.799) (width 1) (layer "F.Cu") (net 3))
 (segment (start 105.918 109.35) (end 104.521 109.35) (width 1) (layer "F.Cu") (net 3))
 (segment (start 125.5649 141.989) (end 132.458 141.989) (width 1) (layer "F.Cu") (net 3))
 (segment (start 140.846 141.989) (end 143.637 144.78) (width 1) (layer "F.Cu") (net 3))
 (segment (start 147.94 161.278) (end 149.606 161.278) (width 1) (layer "F.Cu") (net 3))
 (segment (start 109.256479 137.453479) (end 113.792 141.989) (width 1) (layer "F.Cu") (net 3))
 (segment (start 138.938 135.509) (end 140.84 135.509) (width 1) (layer "F.Cu") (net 3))
 (segment (start 103.378 108.207) (end 103.251 108.08) (width 1) (layer "F.Cu") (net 3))
 (segment (start 132.458 141.989) (end 138.938 135.509) (width 1) (layer "F.Cu") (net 3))
 (segment (start 140.843 141.989) (end 140.846 141.989) (width 1) (layer "F.Cu") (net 3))
 (segment (start 154.813 121.542) (end 153.289 121.542) (width 1) (layer "F.Cu") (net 3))
 (segment (start 140.843 135.512) (end 140.843 141.989) (width 1) (layer "F.Cu") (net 3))
 (via (at 140.843 135.512) (size 2) (drill 1.5) (layers "F.Cu" "B.Cu") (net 3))
 (segment (start 154.813 121.542) (end 140.843 135.512) (width 1) (layer "B.Cu") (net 3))
 (segment (start 96.774 90.808) (end 101.219 95.253) (width 1) (layer "F.Cu") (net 13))
 (segment (start 101.378 68.678) (end 96.774 73.282) (width 1) (layer "F.Cu") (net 13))
 (segment (start 96.774 73.282) (end 96.774 90.808) (width 1) (layer "F.Cu") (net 13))
 (segment (start 101.378 49.882) (end 101.378 68.678) (width 1) (layer "F.Cu") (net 13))
 (segment (start 101.346 39.881) (end 101.346 49.85) (width 1) (layer "F.Cu") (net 13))
 (segment (start 101.346 49.85) (end 101.378 49.882) (width 1) (layer "F.Cu") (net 13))
 (segment (start 110.776 49.882) (end 114.776 49.882) (width 1) (layer "F.Cu") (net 17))
 (segment (start 114.776 49.882) (end 125.698 60.804) (width 1) (layer "F.Cu") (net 17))
 (segment (start 106.1405 49.8185) (end 106.077 49.882) (width 1) (layer "F.Cu") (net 16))
 (segment (start 106.1405 39.595) (end 106.1405 49.8185) (width 1) (layer "F.Cu") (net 16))
 (segment (start 101.219 113.033) (end 104.14 115.954) (width 0.25) (layer "B.Cu") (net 19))
 (segment (start 104.902 121.415) (end 104.14 120.653) (width 0.25) (layer "B.Cu") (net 19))
 (segment (start 105.918 121.415) (end 104.902 121.415) (width 0.25) (layer "B.Cu") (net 19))
 (segment (start 104.14 115.954) (end 104.14 116.078) (width 0.25) (layer "B.Cu") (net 19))
 (segment (start 104.14 120.653) (end 104.14 116.078) (width 0.25) (layer "B.Cu") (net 19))
 (segment (start 110.998 131.445) (end 98.679 143.764) (width 0.25) (layer "B.Cu") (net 14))
 (segment (start 110.998 115.951) (end 110.998 131.445) (width 0.25) (layer "B.Cu") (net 14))
 (segment (start 119.507 107.442) (end 110.998 115.951) (width 0.25) (layer "B.Cu") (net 14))
 (segment (start 98.679 143.764) (end 98.679 146.053) (width 0.25) (layer "B.Cu") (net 14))
 (segment (start 127.095 88.046) (end 132.588 82.553) (width 0.25) (layer "B.Cu") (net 6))
 (segment (start 132.588 82.553) (end 159.639 82.553) (width 0.25) (layer "B.Cu") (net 6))
 (segment (start 157.734 110.493) (end 154.813 113.414) (width 0.25) (layer "B.Cu") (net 34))
 (segment (start 162.179 110.493) (end 157.734 110.493) (width 0.25) (layer "B.Cu") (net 34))
 (segment (start 154.813 113.414) (end 154.813 116.462) (width 0.25) (layer "B.Cu") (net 34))
 (segment (start 130.175 144.0591) (end 130.175 139.068) (width 0.25) (layer "B.Cu") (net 29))
 (segment (start 130.175 139.068) (end 132.08 137.163) (width 0.25) (layer "B.Cu") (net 29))
 (segment (start 162.179 125.733) (end 150.749 137.163) (width 0.25) (layer "B.Cu") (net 29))
 (segment (start 132.08 137.163) (end 150.749 137.163) (width 0.25) (layer "B.Cu") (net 29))
 (segment (start 146.939 164.468) (end 146.939 167.643) (width 0.25) (layer "B.Cu") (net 32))
 (segment (start 148.082 168.786) (end 152.527 168.786) (width 0.25) (layer "B.Cu") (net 32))
 (segment (start 164.433489 134.718489) (end 160.813511 134.718489) (width 0.25) (layer "B.Cu") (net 32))
 (segment (start 129.3749 152.149) (end 134.62 152.149) (width 0.25) (layer "B.Cu") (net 32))
 (segment (start 165.1 135.385) (end 164.433489 134.718489) (width 0.25) (layer "B.Cu") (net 32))
 (segment (start 165.1 156.213) (end 165.1 135.385) (width 0.25) (layer "B.Cu") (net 32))
 (segment (start 160.813511 134.718489) (end 159.639 135.893) (width 0.25) (layer "B.Cu") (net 32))
 (segment (start 146.939 167.643) (end 148.082 168.786) (width 0.25) (layer "B.Cu") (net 32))
 (segment (start 134.62 152.149) (end 146.939 164.468) (width 0.25) (layer "B.Cu") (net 32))
 (segment (start 152.527 168.786) (end 165.1 156.213) (width 0.25) (layer "B.Cu") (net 32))
 (segment (start 123.825 146.5991) (end 129.3749 152.149) (width 0.25) (layer "B.Cu") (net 32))
 (segment (start 126.365 146.5991) (end 131.2799 151.514) (width 0.25) (layer "B.Cu") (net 30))
 (segment (start 147.574 167.262) (end 148.463 168.151) (width 0.25) (layer "B.Cu") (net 30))
 (segment (start 147.574 164.341) (end 147.574 167.262) (width 0.25) (layer "B.Cu") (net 30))
 (segment (start 131.2799 151.514) (end 134.747 151.514) (width 0.25) (layer "B.Cu") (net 30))
 (segment (start 152.273 168.151) (end 164.465 155.959) (width 0.25) (layer "B.Cu") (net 30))
 (segment (start 164.465 155.959) (end 164.465 138.557) (width 0.25) (layer "B.Cu") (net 30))
 (segment (start 134.747 151.514) (end 147.574 164.341) (width 0.25) (layer "B.Cu") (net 30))
 (segment (start 162.179 135.893) (end 164.465 138.179) (width 0.25) (layer "B.Cu") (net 30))
 (segment (start 148.463 168.151) (end 152.273 168.151) (width 0.25) (layer "B.Cu") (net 30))
 (segment (start 164.465 138.179) (end 164.465 138.557) (width 0.25) (layer "B.Cu") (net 30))
 (segment (start 159.044479 137.838479) (end 159.639 138.433) (width 0.25) (layer "B.Cu") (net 31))
 (segment (start 126.3269 145.291) (end 131.191 145.291) (width 0.25) (layer "B.Cu") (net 31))
 (segment (start 131.572 144.91) (end 131.572 138.941) (width 0.25) (layer "B.Cu") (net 31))
 (segment (start 131.191 145.291) (end 131.572 144.91) (width 0.25) (layer "B.Cu") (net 31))
 (segment (start 132.674521 137.838479) (end 159.044479 137.838479) (width 0.25) (layer "B.Cu") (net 31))
 (segment (start 125.095 144.0591) (end 126.3269 145.291) (width 0.25) (layer "B.Cu") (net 31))
 (segment (start 131.572 138.941) (end 132.674521 137.838479) (width 0.25) (layer "B.Cu") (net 31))
 (segment (start 152.542 166.358) (end 149.606 166.358) (width 0.25) (layer "B.Cu") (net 1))
 (segment (start 158.623 153.546) (end 158.115 154.054) (width 0.25) (layer "B.Cu") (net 1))
 (segment (start 163.576 151.768) (end 161.798 153.546) (width 0.25) (layer "B.Cu") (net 1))
 (segment (start 162.687 138.433) (end 163.576 139.322) (width 0.25) (layer "B.Cu") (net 1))
 (segment (start 162.179 138.433) (end 162.687 138.433) (width 0.25) (layer "B.Cu") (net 1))
 (segment (start 158.115 160.785) (end 152.542 166.358) (width 0.25) (layer "B.Cu") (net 1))
 (segment (start 161.798 153.546) (end 158.623 153.546) (width 0.25) (layer "B.Cu") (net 1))
 (segment (start 158.115 154.054) (end 158.115 160.785) (width 0.25) (layer "B.Cu") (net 1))
 (segment (start 163.576 139.322) (end 163.576 151.768) (width 0.25) (layer "B.Cu") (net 1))
 (segment (start 136.909 139.8651) (end 150.4031 139.8651) (width 0.25) (layer "B.Cu") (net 27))
 (segment (start 158.623 141.989) (end 159.639 140.973) (width 0.25) (layer "B.Cu") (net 27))
 (segment (start 150.4031 139.8651) (end 152.527 141.989) (width 0.25) (layer "B.Cu") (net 27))
 (segment (start 132.715 144.0591) (end 136.909 139.8651) (width 0.25) (layer "B.Cu") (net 27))
 (segment (start 152.527 141.989) (end 158.623 141.989) (width 0.25) (layer "B.Cu") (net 27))
 (segment (start 131.445 146.5991) (end 137.7569 152.911) (width 0.25) (layer "B.Cu") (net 28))
 (segment (start 161.163 152.911) (end 162.179 151.895) (width 0.25) (layer "B.Cu") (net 28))
 (segment (start 137.7569 152.911) (end 161.163 152.911) (width 0.25) (layer "B.Cu") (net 28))
 (segment (start 162.179 151.895) (end 162.179 140.973) (width 0.25) (layer "B.Cu") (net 28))
 (segment (start 156.083 135.255) (end 156.083 139.957) (width 0.25) (layer "F.Cu") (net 15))
 (segment (start 119.507 109.982) (end 143.637 134.112) (width 0.25) (layer "F.Cu") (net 15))
 (segment (start 143.637 134.112) (end 154.94 134.112) (width 0.25) (layer "F.Cu") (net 15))
 (segment (start 154.94 134.112) (end 156.083 135.255) (width 0.25) (layer "F.Cu") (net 15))
 (segment (start 156.083 139.957) (end 159.639 143.513) (width 0.25) (layer "F.Cu") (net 15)))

